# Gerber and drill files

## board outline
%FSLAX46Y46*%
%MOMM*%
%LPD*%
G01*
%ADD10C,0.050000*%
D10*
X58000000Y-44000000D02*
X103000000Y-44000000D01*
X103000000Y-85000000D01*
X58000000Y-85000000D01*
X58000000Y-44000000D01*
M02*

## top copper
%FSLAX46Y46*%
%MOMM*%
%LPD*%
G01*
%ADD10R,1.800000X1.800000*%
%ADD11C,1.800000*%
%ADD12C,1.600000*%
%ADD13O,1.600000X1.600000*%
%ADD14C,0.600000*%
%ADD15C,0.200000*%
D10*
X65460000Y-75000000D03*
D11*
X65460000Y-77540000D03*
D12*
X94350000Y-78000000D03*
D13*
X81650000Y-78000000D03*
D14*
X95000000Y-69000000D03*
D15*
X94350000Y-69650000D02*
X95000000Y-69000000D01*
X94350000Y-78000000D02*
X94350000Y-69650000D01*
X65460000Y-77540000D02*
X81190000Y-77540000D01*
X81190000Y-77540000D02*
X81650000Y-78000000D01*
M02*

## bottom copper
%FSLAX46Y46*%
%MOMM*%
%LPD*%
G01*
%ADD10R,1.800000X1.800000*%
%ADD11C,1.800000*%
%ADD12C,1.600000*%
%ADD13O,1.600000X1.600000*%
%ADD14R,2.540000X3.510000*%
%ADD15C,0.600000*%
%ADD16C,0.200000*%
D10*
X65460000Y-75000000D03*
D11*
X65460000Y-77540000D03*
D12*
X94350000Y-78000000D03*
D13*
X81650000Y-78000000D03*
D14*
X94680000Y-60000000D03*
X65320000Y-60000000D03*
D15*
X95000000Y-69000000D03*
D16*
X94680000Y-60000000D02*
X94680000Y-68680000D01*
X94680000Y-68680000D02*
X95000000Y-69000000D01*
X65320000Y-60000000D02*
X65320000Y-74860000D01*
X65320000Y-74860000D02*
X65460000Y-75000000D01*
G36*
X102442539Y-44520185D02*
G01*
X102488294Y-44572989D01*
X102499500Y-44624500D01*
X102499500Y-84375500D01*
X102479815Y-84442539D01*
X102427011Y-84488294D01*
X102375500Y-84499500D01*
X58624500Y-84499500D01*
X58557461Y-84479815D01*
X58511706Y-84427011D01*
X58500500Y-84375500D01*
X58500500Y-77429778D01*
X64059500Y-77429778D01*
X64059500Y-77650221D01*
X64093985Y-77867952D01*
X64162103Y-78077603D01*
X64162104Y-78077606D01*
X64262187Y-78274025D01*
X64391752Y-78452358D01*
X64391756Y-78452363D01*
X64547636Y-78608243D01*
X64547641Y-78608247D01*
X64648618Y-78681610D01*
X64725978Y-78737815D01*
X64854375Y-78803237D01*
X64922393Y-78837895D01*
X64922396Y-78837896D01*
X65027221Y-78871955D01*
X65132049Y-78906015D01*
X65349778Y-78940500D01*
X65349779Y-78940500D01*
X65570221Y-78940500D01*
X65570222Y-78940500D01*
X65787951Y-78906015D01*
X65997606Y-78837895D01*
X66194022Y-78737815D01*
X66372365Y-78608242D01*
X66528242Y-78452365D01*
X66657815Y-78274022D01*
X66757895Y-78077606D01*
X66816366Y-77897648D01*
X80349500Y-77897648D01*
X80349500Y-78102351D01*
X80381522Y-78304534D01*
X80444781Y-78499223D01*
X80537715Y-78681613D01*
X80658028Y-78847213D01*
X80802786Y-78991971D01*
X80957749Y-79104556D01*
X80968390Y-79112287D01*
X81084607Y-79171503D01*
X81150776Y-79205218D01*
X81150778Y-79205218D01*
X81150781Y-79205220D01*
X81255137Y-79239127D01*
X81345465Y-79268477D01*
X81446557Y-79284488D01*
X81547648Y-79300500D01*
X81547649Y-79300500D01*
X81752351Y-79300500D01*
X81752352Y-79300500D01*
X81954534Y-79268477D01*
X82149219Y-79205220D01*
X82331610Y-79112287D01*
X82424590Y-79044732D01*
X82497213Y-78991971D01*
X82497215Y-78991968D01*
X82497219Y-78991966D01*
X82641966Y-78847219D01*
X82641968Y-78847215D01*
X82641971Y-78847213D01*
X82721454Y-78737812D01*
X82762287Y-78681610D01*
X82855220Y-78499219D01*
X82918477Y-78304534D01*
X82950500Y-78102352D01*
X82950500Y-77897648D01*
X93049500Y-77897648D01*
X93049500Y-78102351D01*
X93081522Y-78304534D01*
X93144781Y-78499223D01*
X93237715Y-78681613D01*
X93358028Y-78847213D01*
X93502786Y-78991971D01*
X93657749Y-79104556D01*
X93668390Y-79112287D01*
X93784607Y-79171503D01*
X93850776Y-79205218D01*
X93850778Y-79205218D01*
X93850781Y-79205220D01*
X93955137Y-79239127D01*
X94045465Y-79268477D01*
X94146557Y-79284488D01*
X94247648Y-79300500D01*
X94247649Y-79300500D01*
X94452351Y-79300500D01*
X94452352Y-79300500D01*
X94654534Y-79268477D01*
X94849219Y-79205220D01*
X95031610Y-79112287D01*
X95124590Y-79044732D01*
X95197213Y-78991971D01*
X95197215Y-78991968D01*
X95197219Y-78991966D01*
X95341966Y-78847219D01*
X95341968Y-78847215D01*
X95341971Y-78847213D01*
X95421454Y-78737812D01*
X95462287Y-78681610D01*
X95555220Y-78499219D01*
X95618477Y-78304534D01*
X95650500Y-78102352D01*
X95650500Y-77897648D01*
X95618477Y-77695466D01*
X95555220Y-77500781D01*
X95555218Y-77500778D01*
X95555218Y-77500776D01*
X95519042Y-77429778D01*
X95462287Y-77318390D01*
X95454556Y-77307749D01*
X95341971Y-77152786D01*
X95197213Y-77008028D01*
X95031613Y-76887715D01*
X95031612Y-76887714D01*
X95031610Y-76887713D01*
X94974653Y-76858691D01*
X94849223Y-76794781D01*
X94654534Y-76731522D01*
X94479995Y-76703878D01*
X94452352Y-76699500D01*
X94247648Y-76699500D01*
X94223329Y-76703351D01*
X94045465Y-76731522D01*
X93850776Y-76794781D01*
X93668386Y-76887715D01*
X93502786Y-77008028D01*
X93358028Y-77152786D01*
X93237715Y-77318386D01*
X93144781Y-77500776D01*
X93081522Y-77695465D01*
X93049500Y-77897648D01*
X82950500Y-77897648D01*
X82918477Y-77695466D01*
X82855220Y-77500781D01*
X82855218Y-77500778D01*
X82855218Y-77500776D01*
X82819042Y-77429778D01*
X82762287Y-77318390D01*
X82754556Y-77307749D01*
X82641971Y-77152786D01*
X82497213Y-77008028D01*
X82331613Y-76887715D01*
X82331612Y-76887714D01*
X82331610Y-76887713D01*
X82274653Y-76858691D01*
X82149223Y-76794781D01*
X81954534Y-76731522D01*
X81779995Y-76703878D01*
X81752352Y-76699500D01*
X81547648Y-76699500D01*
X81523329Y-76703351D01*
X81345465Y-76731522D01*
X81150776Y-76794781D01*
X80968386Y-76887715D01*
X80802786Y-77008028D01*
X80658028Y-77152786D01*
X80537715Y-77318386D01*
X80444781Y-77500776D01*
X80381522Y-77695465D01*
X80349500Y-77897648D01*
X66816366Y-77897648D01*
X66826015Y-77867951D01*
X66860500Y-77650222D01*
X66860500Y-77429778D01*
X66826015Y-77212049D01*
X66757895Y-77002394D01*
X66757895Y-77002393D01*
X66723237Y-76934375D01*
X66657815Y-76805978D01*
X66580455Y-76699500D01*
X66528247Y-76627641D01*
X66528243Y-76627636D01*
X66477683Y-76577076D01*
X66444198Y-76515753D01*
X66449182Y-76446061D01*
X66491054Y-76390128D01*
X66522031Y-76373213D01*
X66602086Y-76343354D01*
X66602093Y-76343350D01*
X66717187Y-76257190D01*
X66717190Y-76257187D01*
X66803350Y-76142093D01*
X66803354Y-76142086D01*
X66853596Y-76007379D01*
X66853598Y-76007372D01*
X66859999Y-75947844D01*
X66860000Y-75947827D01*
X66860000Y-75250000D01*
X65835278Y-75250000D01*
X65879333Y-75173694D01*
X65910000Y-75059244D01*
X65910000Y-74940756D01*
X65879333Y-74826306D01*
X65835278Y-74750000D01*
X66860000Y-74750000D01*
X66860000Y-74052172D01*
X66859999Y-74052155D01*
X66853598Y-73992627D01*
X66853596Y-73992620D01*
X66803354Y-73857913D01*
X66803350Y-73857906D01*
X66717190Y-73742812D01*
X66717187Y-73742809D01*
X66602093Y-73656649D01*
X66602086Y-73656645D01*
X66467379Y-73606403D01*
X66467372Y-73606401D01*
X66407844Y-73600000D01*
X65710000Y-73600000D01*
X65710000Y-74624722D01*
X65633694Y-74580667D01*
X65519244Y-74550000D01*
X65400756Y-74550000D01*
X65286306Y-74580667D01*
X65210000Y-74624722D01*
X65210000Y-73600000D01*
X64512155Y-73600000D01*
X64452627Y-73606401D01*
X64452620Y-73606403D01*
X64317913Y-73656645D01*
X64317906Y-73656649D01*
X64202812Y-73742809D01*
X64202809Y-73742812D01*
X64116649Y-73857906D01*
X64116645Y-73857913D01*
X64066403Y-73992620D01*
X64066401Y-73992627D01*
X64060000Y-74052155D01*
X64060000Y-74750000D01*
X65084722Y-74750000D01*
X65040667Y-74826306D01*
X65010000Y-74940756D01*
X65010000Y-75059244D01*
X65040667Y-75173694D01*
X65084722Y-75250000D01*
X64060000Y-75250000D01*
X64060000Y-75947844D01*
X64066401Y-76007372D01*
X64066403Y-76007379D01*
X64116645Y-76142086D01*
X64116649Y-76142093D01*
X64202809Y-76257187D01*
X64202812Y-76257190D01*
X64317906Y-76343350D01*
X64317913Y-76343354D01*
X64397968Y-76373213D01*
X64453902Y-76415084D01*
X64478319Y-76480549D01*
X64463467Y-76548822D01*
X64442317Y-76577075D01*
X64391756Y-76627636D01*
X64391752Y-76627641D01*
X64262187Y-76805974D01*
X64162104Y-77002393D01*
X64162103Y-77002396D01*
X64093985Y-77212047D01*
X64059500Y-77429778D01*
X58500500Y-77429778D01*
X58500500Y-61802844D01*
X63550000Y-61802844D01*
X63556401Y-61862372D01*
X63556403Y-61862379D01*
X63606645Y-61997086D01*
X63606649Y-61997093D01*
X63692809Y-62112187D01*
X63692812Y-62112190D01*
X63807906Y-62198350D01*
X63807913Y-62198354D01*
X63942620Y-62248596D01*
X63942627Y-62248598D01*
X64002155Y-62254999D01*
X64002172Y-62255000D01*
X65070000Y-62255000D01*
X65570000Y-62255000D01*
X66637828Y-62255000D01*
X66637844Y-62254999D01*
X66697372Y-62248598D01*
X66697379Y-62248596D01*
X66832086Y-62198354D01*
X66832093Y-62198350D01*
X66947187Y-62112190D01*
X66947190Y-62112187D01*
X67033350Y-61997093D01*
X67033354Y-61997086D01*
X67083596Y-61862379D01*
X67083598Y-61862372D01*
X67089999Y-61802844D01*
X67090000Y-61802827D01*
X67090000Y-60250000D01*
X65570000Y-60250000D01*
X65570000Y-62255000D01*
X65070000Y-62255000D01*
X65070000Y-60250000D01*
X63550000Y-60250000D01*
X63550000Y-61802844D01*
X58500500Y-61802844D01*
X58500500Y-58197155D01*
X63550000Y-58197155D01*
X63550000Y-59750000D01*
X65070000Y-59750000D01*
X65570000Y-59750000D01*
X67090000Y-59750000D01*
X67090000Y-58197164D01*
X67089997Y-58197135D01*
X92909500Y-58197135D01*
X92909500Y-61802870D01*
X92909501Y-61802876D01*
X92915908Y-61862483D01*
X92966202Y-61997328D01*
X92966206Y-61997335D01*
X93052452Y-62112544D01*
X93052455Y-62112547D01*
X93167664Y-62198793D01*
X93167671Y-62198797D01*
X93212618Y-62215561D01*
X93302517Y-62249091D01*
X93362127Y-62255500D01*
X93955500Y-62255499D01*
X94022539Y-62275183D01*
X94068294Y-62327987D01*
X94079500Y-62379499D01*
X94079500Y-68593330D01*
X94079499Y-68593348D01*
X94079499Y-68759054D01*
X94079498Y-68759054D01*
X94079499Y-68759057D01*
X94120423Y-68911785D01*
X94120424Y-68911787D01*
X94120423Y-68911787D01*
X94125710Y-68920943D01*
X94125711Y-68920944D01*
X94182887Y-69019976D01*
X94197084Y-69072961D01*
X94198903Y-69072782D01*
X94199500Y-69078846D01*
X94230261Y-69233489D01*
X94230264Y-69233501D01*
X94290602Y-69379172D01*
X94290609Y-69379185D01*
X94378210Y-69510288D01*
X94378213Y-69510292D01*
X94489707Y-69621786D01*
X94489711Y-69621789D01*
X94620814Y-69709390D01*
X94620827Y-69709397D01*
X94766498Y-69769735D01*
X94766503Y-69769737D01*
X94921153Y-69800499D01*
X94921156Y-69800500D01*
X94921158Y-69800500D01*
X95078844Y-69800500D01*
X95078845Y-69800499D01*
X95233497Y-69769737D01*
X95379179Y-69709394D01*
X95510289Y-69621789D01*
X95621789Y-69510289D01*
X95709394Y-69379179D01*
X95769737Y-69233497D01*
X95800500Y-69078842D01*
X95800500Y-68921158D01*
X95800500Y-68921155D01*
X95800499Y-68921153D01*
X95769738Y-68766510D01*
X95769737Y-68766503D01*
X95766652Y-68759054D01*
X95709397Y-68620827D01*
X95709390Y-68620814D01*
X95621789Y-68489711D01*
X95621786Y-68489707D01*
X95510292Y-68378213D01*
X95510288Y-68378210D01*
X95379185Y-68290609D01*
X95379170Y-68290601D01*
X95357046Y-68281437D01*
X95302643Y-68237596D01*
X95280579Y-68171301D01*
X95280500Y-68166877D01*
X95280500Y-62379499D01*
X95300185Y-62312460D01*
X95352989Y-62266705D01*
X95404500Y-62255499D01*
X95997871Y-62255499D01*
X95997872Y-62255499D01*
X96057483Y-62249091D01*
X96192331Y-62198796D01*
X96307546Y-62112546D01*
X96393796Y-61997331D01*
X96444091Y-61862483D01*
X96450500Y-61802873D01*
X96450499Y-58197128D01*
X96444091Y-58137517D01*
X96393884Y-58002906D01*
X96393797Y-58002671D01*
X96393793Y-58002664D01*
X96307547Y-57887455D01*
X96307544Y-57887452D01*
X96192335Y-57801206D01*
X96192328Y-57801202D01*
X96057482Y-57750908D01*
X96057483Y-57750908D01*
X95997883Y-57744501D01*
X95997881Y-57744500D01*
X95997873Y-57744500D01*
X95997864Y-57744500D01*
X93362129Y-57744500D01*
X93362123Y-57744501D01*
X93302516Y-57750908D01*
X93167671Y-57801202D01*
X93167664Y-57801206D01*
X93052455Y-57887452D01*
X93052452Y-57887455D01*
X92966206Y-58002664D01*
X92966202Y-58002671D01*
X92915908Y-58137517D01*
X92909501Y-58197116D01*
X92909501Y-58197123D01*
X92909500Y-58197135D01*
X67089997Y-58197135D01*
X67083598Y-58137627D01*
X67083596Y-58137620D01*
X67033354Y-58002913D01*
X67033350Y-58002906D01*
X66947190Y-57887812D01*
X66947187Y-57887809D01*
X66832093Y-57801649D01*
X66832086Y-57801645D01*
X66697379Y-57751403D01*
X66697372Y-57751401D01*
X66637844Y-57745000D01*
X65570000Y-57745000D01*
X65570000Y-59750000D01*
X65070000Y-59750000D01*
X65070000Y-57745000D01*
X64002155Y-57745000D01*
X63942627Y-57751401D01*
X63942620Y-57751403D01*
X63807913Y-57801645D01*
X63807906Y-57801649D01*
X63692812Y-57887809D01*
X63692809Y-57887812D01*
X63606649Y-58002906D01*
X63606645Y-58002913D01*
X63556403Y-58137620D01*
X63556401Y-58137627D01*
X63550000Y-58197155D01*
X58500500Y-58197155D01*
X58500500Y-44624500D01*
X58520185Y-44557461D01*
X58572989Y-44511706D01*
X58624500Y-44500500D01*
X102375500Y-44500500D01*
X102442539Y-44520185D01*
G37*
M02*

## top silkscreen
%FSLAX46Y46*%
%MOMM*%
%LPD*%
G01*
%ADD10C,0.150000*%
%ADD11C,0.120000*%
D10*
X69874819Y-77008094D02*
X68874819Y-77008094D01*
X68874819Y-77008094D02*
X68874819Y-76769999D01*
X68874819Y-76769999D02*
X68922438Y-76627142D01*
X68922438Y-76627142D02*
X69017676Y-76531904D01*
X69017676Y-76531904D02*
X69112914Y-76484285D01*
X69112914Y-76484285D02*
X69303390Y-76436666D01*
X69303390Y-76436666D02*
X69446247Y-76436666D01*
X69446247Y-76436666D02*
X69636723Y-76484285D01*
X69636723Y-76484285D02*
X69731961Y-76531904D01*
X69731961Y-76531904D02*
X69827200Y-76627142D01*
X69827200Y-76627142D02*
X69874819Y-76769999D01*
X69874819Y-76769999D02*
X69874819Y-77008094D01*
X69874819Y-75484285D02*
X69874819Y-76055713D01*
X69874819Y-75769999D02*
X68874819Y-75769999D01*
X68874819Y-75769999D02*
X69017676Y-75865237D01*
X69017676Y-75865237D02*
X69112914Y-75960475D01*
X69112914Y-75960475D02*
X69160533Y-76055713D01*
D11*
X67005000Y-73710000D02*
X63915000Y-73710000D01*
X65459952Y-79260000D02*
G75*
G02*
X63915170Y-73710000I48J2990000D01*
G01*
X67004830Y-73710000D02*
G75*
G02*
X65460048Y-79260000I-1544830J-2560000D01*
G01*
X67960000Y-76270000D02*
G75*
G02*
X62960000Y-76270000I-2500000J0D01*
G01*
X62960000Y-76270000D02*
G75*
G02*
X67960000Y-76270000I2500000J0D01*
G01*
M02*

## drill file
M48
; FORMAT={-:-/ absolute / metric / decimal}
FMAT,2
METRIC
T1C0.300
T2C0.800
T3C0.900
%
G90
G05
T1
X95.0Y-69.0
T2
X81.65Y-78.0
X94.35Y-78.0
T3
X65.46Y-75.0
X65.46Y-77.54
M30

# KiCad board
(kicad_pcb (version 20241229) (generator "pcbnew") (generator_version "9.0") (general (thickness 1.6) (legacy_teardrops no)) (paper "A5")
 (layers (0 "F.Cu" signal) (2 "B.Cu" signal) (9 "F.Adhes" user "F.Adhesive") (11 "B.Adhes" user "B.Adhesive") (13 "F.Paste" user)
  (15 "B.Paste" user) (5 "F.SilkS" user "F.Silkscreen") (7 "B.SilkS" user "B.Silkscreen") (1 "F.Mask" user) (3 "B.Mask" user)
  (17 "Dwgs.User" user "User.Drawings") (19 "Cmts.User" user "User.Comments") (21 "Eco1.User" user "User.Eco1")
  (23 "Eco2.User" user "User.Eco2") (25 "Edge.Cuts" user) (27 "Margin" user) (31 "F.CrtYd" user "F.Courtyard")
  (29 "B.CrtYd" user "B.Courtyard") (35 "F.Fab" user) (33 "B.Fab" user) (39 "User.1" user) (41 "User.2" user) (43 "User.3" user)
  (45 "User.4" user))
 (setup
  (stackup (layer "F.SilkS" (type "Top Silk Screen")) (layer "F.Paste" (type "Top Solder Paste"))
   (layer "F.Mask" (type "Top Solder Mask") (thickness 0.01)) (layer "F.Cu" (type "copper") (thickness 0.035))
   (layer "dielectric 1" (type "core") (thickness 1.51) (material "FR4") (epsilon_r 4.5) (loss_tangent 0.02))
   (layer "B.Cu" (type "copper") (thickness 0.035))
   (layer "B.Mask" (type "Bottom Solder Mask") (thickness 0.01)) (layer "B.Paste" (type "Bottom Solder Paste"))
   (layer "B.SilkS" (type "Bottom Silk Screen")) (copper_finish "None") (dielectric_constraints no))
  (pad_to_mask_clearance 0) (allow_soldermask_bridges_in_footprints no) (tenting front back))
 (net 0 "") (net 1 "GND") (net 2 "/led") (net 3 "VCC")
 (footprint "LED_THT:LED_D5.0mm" (layer "F.Cu") (at 65.46 75 -90)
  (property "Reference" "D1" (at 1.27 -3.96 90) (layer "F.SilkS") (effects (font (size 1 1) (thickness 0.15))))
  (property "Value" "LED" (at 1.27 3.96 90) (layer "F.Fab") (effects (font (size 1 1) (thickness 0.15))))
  (fp_line (start -1.29 -1.545) (end -1.29 1.545) (stroke (width 0.12) (type solid)) (layer "F.SilkS"))
  (fp_arc (start 4.26 0.000048) (mid 2.071756 2.880501) (end -1.29 1.54483) (stroke (width 0.12) (type solid)) (layer "F.SilkS"))
  (fp_arc (start -1.29 -1.54483) (mid 2.071756 -2.880501) (end 4.26 -0.000048) (stroke (width 0.12) (type solid)) (layer "F.SilkS"))
  (fp_circle (center 1.27 0) (end 3.77 0) (stroke (width 0.12) (type solid)) (fill no) (layer "F.SilkS"))
  (pad "1" thru_hole rect (at 0 0 270) (size 1.8 1.8) (drill 0.9) (layers "*.Cu" "*.Mask") (remove_unused_layers no) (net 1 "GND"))
  (pad "2" thru_hole circle (at 2.54 0 270) (size 1.8 1.8) (drill 0.9) (layers "*.Cu" "*.Mask") (remove_unused_layers no) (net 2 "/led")))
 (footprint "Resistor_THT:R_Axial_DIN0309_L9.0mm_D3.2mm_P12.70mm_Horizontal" (layer "B.Cu") (at 94.35 78 180)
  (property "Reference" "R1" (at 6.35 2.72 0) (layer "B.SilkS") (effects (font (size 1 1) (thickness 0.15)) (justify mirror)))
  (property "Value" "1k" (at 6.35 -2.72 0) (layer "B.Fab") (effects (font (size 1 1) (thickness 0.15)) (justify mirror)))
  (pad "1" thru_hole circle (at 0 0 180) (size 1.6 1.6) (drill 0.8) (layers "*.Cu" "*.Mask") (remove_unused_layers no) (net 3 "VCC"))
  (pad "2" thru_hole oval (at 12.7 0 180) (size 1.6 1.6) (drill 0.8) (layers "*.Cu" "*.Mask") (remove_unused_layers no) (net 2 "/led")))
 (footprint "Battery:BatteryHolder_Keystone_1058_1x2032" (layer "B.Cu") (at 80 60 180)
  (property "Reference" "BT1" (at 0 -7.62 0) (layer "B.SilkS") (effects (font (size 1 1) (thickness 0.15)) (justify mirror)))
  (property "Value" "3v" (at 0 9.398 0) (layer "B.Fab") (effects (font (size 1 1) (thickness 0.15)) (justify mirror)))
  (pad "1" smd rect (at -14.68 0 180) (size 2.54 3.51) (layers "B.Cu" "B.Mask" "B.Paste") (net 3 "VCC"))
  (pad "2" smd rect (at 14.68 0 180) (size 2.54 3.51) (layers "B.Cu" "B.Mask" "B.Paste") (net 1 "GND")))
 (gr_rect (start 58 44) (end 103 85) (stroke (width 0.05) (type default)) (fill no) (layer "Edge.Cuts"))
 (segment (start 94.35 69.65) (end 95 69) (width 0.2) (layer "F.Cu") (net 3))
 (segment (start 94.35 78) (end 94.35 69.65) (width 0.2) (layer "F.Cu") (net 3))
 (via (at 95 69) (size 0.6) (drill 0.3) (layers "F.Cu" "B.Cu") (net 3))
 (segment (start 94.68 60) (end 94.68 68.68) (width 0.2) (layer "B.Cu") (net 3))
 (segment (start 94.68 68.68) (end 95 69) (width 0.2) (layer "B.Cu") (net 3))
 (segment (start 65.32 60) (end 65.32 74.86) (width 0.2) (layer "B.Cu") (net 1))
 (segment (start 65.32 74.86) (end 65.46 75) (width 0.2) (layer "B.Cu") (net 1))
 (segment (start 65.46 77.54) (end 81.19 77.54) (width 0.2) (layer "F.Cu") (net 2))
 (segment (start 81.19 77.54) (end 81.65 78) (width 0.2) (layer "F.Cu") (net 2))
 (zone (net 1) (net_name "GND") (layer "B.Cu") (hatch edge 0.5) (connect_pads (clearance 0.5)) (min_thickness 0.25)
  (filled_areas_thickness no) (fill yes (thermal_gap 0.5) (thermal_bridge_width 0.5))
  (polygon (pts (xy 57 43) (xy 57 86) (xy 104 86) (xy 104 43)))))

